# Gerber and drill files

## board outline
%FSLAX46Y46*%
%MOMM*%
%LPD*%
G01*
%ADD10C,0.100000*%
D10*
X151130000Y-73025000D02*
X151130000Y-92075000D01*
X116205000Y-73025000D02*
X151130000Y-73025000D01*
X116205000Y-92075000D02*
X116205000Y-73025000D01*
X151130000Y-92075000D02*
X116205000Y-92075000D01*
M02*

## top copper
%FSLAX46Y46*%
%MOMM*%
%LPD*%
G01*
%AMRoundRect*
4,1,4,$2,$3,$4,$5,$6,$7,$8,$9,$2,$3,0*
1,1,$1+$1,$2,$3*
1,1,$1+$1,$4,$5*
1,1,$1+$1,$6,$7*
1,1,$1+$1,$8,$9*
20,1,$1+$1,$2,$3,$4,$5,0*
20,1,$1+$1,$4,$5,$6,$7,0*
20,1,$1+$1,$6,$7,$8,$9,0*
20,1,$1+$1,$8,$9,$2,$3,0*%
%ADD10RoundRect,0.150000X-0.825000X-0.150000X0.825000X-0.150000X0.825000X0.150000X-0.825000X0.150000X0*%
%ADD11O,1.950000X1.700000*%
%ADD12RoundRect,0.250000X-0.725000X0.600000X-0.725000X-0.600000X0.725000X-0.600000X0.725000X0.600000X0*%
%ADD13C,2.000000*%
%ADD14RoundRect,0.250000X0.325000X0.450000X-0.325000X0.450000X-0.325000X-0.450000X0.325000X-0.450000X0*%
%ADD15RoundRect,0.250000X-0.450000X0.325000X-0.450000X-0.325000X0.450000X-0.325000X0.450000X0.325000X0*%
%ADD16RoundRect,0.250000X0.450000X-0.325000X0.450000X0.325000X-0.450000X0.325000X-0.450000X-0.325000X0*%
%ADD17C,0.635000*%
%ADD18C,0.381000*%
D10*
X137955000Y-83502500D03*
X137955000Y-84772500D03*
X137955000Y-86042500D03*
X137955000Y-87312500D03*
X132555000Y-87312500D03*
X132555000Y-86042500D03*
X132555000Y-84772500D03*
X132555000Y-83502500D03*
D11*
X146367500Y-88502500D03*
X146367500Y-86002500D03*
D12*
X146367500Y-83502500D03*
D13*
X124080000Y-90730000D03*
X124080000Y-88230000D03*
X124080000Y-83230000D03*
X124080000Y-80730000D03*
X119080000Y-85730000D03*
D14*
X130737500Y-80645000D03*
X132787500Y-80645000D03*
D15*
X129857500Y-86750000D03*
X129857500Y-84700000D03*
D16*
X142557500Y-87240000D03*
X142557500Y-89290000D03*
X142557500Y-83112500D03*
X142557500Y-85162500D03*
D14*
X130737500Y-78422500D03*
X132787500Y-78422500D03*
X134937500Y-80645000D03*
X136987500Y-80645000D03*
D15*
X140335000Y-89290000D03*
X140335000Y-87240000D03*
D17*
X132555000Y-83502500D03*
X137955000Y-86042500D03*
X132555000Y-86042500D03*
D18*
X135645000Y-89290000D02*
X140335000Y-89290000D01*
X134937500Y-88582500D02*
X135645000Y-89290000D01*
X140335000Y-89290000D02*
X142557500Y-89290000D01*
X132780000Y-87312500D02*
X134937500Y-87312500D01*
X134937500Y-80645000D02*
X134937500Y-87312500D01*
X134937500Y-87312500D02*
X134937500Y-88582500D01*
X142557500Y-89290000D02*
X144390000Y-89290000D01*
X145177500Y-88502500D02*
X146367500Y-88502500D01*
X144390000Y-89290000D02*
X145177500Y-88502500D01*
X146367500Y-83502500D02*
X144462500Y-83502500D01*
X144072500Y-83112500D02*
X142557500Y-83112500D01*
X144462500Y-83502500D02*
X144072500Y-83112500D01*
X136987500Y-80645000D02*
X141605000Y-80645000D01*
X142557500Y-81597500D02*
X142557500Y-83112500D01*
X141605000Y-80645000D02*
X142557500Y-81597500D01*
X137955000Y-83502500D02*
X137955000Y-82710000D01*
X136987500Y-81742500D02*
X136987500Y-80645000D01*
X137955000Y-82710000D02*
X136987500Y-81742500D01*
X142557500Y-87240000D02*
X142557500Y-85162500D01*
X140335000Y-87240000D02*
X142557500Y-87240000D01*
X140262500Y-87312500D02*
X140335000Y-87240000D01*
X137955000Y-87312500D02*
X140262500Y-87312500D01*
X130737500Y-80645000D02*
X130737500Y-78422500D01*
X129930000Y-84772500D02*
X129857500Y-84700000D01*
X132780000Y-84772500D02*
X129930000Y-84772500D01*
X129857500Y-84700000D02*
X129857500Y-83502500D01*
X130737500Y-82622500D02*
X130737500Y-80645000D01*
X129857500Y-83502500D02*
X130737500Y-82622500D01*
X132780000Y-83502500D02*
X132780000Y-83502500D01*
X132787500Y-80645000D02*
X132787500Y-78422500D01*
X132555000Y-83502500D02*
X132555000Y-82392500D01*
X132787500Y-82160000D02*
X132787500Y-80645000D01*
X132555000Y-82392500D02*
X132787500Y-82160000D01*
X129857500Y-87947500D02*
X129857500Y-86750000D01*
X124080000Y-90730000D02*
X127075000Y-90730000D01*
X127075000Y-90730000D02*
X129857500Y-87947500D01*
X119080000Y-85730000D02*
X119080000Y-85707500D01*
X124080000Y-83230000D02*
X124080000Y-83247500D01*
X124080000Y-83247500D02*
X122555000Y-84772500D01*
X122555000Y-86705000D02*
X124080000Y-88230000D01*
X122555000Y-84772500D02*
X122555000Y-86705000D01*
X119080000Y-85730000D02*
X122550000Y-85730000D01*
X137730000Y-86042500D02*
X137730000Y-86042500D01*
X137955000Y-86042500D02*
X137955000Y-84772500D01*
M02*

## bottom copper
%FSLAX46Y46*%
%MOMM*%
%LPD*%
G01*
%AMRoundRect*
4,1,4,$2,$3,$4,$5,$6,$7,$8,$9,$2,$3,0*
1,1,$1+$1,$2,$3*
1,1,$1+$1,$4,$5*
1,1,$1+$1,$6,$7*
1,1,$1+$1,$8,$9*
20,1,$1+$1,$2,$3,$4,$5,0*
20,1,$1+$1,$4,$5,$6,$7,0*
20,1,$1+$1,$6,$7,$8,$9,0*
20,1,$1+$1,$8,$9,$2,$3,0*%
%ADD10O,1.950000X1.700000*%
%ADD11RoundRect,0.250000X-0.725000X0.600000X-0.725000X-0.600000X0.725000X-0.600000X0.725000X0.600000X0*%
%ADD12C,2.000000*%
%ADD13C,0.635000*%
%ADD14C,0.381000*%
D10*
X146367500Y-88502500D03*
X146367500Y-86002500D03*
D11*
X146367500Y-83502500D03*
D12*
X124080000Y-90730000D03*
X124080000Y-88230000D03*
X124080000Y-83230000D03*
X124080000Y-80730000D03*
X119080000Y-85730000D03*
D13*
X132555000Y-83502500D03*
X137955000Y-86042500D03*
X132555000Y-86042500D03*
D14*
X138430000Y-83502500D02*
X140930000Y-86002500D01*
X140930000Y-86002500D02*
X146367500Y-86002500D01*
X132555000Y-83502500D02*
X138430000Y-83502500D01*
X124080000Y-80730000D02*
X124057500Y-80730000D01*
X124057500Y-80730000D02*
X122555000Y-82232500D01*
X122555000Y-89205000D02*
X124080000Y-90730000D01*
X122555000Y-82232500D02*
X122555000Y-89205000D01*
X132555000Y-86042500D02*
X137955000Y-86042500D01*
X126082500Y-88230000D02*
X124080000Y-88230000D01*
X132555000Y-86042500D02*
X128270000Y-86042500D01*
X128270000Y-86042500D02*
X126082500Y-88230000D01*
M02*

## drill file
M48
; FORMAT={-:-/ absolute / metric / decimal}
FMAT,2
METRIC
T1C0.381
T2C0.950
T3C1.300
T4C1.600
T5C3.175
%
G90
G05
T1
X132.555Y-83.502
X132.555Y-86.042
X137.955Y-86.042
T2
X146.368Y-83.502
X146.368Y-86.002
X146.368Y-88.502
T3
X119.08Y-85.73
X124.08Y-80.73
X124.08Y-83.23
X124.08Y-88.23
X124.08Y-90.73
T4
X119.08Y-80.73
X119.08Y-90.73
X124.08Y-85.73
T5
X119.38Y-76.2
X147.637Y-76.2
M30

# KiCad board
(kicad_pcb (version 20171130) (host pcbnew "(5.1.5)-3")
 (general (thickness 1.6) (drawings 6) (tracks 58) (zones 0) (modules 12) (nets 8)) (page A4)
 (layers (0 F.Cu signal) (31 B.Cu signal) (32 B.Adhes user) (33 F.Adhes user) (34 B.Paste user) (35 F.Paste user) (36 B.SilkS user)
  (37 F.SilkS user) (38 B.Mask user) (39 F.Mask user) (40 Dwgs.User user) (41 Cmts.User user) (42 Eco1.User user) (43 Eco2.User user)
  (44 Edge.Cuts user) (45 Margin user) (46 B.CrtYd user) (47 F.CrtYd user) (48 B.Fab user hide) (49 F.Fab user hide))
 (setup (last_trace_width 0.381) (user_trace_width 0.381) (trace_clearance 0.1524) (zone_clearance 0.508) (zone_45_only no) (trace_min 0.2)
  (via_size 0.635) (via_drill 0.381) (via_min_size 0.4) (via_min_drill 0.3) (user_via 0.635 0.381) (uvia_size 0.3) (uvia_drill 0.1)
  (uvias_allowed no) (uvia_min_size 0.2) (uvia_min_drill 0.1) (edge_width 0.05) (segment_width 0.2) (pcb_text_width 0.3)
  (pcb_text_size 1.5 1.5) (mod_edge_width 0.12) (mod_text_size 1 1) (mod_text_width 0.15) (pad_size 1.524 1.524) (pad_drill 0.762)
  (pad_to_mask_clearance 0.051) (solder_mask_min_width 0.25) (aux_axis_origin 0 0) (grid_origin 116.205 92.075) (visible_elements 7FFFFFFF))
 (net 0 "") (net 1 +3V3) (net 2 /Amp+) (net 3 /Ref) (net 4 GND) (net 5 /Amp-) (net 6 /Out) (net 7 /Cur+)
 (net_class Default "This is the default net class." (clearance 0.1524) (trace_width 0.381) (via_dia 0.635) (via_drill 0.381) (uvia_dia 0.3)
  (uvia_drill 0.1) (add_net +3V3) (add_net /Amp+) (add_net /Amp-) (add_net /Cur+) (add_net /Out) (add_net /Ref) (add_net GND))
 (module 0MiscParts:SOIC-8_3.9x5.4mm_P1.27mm (layer F.Cu) (at 135.255 85.4075)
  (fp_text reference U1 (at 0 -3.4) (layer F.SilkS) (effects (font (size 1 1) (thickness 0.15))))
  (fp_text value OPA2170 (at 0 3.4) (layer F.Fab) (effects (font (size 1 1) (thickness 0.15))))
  (pad 8 smd roundrect (at 2.7 -1.905) (size 1.95 0.6) (layers F.Cu F.Paste F.Mask) (roundrect_rratio 0.25) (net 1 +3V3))
  (pad 7 smd roundrect (at 2.7 -0.635) (size 1.95 0.6) (layers F.Cu F.Paste F.Mask) (roundrect_rratio 0.25) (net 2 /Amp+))
  (pad 6 smd roundrect (at 2.7 0.635) (size 1.95 0.6) (layers F.Cu F.Paste F.Mask) (roundrect_rratio 0.25) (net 2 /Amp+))
  (pad 5 smd roundrect (at 2.7 1.905) (size 1.95 0.6) (layers F.Cu F.Paste F.Mask) (roundrect_rratio 0.25) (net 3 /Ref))
  (pad 4 smd roundrect (at -2.7 1.905) (size 1.95 0.6) (layers F.Cu F.Paste F.Mask) (roundrect_rratio 0.25) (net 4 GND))
  (pad 3 smd roundrect (at -2.7 0.635) (size 1.95 0.6) (layers F.Cu F.Paste F.Mask) (roundrect_rratio 0.25) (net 2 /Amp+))
  (pad 2 smd roundrect (at -2.7 -0.635) (size 1.95 0.6) (layers F.Cu F.Paste F.Mask) (roundrect_rratio 0.25) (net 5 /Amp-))
  (pad 1 smd roundrect (at -2.7 -1.905) (size 1.95 0.6) (layers F.Cu F.Paste F.Mask) (roundrect_rratio 0.25) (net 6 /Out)))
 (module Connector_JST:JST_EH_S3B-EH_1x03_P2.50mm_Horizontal (layer F.Cu) (at 146.3675 83.5025 270)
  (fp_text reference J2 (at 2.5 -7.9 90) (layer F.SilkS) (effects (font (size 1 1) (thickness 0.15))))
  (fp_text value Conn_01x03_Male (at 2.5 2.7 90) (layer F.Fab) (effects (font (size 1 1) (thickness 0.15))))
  (pad 3 thru_hole oval (at 5 0 270) (size 1.7 1.95) (drill 0.95) (layers *.Cu *.Mask) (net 4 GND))
  (pad 2 thru_hole oval (at 2.5 0 270) (size 1.7 1.95) (drill 0.95) (layers *.Cu *.Mask) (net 6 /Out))
  (pad 1 thru_hole roundrect (at 0 0 270) (size 1.7 1.95) (drill 0.95) (layers *.Cu *.Mask) (roundrect_rratio 0.147059) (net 1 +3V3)))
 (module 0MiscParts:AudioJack (layer F.Cu) (at 119.08 85.73)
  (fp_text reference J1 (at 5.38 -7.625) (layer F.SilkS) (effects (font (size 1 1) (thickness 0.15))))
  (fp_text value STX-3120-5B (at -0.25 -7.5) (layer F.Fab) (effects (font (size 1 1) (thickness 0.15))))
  (pad "" np_thru_hole circle (at 5 0) (size 1.6 1.6) (drill 1.6) (layers *.Cu *.Mask))
  (pad "" np_thru_hole circle (at 0 5) (size 1.6 1.6) (drill 1.6) (layers *.Cu *.Mask))
  (pad "" np_thru_hole circle (at 0 -5) (size 1.6 1.6) (drill 1.6) (layers *.Cu *.Mask))
  (pad 5 thru_hole circle (at 5 5) (size 2 2) (drill 1.3) (layers *.Cu *.Mask) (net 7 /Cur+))
  (pad 4 thru_hole circle (at 5 2.5) (size 2 2) (drill 1.3) (layers *.Cu *.Mask) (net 2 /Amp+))
  (pad 3 thru_hole circle (at 5 -2.5) (size 2 2) (drill 1.3) (layers *.Cu *.Mask) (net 2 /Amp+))
  (pad 2 thru_hole circle (at 5 -5) (size 2 2) (drill 1.3) (layers *.Cu *.Mask) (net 7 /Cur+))
  (pad 1 thru_hole circle (at 0 0) (size 2 2) (drill 1.3) (layers *.Cu *.Mask) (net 2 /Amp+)))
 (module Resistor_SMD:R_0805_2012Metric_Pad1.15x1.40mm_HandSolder (layer F.Cu) (at 131.7625 80.645 180)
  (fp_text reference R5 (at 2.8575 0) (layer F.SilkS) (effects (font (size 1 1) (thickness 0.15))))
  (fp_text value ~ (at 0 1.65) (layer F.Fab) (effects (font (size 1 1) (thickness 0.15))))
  (pad 2 smd roundrect (at 1.025 0 180) (size 1.15 1.4) (layers F.Cu F.Paste F.Mask) (roundrect_rratio 0.217391) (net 5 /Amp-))
  (pad 1 smd roundrect (at -1.025 0 180) (size 1.15 1.4) (layers F.Cu F.Paste F.Mask) (roundrect_rratio 0.217391) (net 6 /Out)))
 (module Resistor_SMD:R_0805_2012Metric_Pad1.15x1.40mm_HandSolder (layer F.Cu) (at 129.8575 85.725 270)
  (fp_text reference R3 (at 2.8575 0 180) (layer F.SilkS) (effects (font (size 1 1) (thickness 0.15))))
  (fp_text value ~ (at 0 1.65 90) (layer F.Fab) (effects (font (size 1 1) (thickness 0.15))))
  (pad 2 smd roundrect (at 1.025 0 270) (size 1.15 1.4) (layers F.Cu F.Paste F.Mask) (roundrect_rratio 0.217391) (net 7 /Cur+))
  (pad 1 smd roundrect (at -1.025 0 270) (size 1.15 1.4) (layers F.Cu F.Paste F.Mask) (roundrect_rratio 0.217391) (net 5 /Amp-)))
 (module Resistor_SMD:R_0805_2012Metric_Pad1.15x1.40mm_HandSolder (layer F.Cu) (at 142.5575 88.265 90)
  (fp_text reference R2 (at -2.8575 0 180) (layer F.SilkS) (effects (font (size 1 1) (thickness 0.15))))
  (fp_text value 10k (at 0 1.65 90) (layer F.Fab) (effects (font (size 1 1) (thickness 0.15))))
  (pad 2 smd roundrect (at 1.025 0 90) (size 1.15 1.4) (layers F.Cu F.Paste F.Mask) (roundrect_rratio 0.217391) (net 3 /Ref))
  (pad 1 smd roundrect (at -1.025 0 90) (size 1.15 1.4) (layers F.Cu F.Paste F.Mask) (roundrect_rratio 0.217391) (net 4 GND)))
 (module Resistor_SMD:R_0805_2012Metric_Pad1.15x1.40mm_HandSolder (layer F.Cu) (at 142.5575 84.1375 90)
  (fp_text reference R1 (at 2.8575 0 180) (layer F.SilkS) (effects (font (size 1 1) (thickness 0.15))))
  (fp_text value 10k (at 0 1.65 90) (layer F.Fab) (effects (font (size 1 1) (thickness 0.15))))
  (pad 2 smd roundrect (at 1.025 0 90) (size 1.15 1.4) (layers F.Cu F.Paste F.Mask) (roundrect_rratio 0.217391) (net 1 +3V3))
  (pad 1 smd roundrect (at -1.025 0 90) (size 1.15 1.4) (layers F.Cu F.Paste F.Mask) (roundrect_rratio 0.217391) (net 3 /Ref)))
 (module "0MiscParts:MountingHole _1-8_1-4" (layer F.Cu) (at 147.6375 76.2)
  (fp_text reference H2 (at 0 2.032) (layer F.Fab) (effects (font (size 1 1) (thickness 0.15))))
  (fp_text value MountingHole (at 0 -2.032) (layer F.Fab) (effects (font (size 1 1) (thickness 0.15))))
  (pad "" np_thru_hole circle (at 0 0) (size 3.175 3.175) (drill 3.175) (layers *.Cu *.Mask)))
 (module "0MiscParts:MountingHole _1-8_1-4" (layer F.Cu) (at 119.38 76.2)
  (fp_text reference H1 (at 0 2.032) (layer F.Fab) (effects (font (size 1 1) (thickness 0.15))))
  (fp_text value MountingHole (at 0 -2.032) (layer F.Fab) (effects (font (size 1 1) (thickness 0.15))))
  (pad "" np_thru_hole circle (at 0 0) (size 3.175 3.175) (drill 3.175) (layers *.Cu *.Mask)))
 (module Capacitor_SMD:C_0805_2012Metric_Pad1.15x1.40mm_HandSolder (layer F.Cu) (at 131.7625 78.4225 180)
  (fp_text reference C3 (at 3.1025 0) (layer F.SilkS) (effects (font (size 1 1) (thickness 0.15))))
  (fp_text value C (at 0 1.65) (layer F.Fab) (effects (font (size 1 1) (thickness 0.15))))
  (pad 2 smd roundrect (at 1.025 0 180) (size 1.15 1.4) (layers F.Cu F.Paste F.Mask) (roundrect_rratio 0.217391) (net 5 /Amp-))
  (pad 1 smd roundrect (at -1.025 0 180) (size 1.15 1.4) (layers F.Cu F.Paste F.Mask) (roundrect_rratio 0.217391) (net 6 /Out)))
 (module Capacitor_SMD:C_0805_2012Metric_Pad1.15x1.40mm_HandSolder (layer F.Cu) (at 135.9625 80.645 180)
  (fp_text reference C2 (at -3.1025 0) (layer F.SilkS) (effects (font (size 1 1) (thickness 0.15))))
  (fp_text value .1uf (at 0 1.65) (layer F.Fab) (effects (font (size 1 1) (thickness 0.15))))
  (pad 2 smd roundrect (at 1.025 0 180) (size 1.15 1.4) (layers F.Cu F.Paste F.Mask) (roundrect_rratio 0.217391) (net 4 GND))
  (pad 1 smd roundrect (at -1.025 0 180) (size 1.15 1.4) (layers F.Cu F.Paste F.Mask) (roundrect_rratio 0.217391) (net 1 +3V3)))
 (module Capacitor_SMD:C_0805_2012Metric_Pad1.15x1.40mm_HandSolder (layer F.Cu) (at 140.335 88.265 270)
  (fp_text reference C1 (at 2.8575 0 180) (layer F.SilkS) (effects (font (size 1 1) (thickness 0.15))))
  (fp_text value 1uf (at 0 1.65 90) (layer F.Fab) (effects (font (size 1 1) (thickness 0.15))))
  (pad 2 smd roundrect (at 1.025 0 270) (size 1.15 1.4) (layers F.Cu F.Paste F.Mask) (roundrect_rratio 0.217391) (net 4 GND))
  (pad 1 smd roundrect (at -1.025 0 270) (size 1.15 1.4) (layers F.Cu F.Paste F.Mask) (roundrect_rratio 0.217391) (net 3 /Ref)))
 (gr_line (start 151.13 73.025) (end 151.13 92.075) (layer Edge.Cuts) (width 0.1))
 (gr_line (start 116.205 73.025) (end 151.13 73.025) (layer Edge.Cuts) (width 0.1))
 (gr_line (start 116.205 92.075) (end 116.205 73.025) (layer Edge.Cuts) (width 0.1))
 (gr_line (start 151.13 92.075) (end 116.205 92.075) (layer Edge.Cuts) (width 0.1))
 (segment (start 135.645 89.29) (end 140.335 89.29) (width 0.381) (layer F.Cu) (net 4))
 (segment (start 134.9375 88.5825) (end 135.645 89.29) (width 0.381) (layer F.Cu) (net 4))
 (segment (start 140.335 89.29) (end 142.5575 89.29) (width 0.381) (layer F.Cu) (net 4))
 (segment (start 132.78 87.3125) (end 134.9375 87.3125) (width 0.381) (layer F.Cu) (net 4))
 (segment (start 134.9375 80.645) (end 134.9375 87.3125) (width 0.381) (layer F.Cu) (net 4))
 (segment (start 134.9375 87.3125) (end 134.9375 88.5825) (width 0.381) (layer F.Cu) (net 4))
 (segment (start 142.5575 89.29) (end 144.39 89.29) (width 0.381) (layer F.Cu) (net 4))
 (segment (start 145.1775 88.5025) (end 146.3675 88.5025) (width 0.381) (layer F.Cu) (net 4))
 (segment (start 144.39 89.29) (end 145.1775 88.5025) (width 0.381) (layer F.Cu) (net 4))
 (segment (start 146.3675 83.5025) (end 144.4625 83.5025) (width 0.381) (layer F.Cu) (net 1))
 (segment (start 144.0725 83.1125) (end 142.5575 83.1125) (width 0.381) (layer F.Cu) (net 1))
 (segment (start 144.4625 83.5025) (end 144.0725 83.1125) (width 0.381) (layer F.Cu) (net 1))
 (segment (start 136.9875 80.645) (end 141.605 80.645) (width 0.381) (layer F.Cu) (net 1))
 (segment (start 142.5575 81.5975) (end 142.5575 83.1125) (width 0.381) (layer F.Cu) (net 1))
 (segment (start 141.605 80.645) (end 142.5575 81.5975) (width 0.381) (layer F.Cu) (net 1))
 (segment (start 137.955 83.5025) (end 137.955 82.71) (width 0.381) (layer F.Cu) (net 1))
 (segment (start 136.9875 81.7425) (end 136.9875 80.645) (width 0.381) (layer F.Cu) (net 1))
 (segment (start 137.955 82.71) (end 136.9875 81.7425) (width 0.381) (layer F.Cu) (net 1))
 (segment (start 142.5575 87.24) (end 142.5575 85.1625) (width 0.381) (layer F.Cu) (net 3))
 (segment (start 140.335 87.24) (end 142.5575 87.24) (width 0.381) (layer F.Cu) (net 3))
 (segment (start 140.2625 87.3125) (end 140.335 87.24) (width 0.381) (layer F.Cu) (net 3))
 (segment (start 137.955 87.3125) (end 140.2625 87.3125) (width 0.381) (layer F.Cu) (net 3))
 (segment (start 130.7375 80.645) (end 130.7375 78.4225) (width 0.381) (layer F.Cu) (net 5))
 (segment (start 129.93 84.7725) (end 129.8575 84.7) (width 0.381) (layer F.Cu) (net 5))
 (segment (start 132.78 84.7725) (end 129.93 84.7725) (width 0.381) (layer F.Cu) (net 5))
 (segment (start 129.8575 84.7) (end 129.8575 83.5025) (width 0.381) (layer F.Cu) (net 5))
 (segment (start 130.7375 82.6225) (end 130.7375 80.645) (width 0.381) (layer F.Cu) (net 5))
 (segment (start 129.8575 83.5025) (end 130.7375 82.6225) (width 0.381) (layer F.Cu) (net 5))
 (segment (start 132.78 83.5025) (end 132.78 83.5025) (width 0.381) (layer F.Cu) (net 6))
 (segment (start 132.7875 80.645) (end 132.7875 78.4225) (width 0.381) (layer F.Cu) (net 6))
 (segment (start 138.43 83.5025) (end 140.93 86.0025) (width 0.381) (layer B.Cu) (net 6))
 (via (at 132.555 83.5025) (size 0.635) (drill 0.381) (layers F.Cu B.Cu) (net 6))
 (segment (start 140.93 86.0025) (end 146.3675 86.0025) (width 0.381) (layer B.Cu) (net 6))
 (segment (start 132.555 83.5025) (end 138.43 83.5025) (width 0.381) (layer B.Cu) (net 6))
 (segment (start 132.555 83.5025) (end 132.555 82.3925) (width 0.381) (layer F.Cu) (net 6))
 (segment (start 132.7875 82.16) (end 132.7875 80.645) (width 0.381) (layer F.Cu) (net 6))
 (segment (start 132.555 82.3925) (end 132.7875 82.16) (width 0.381) (layer F.Cu) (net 6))
 (segment (start 124.08 80.73) (end 124.0575 80.73) (width 0.381) (layer B.Cu) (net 7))
 (segment (start 124.0575 80.73) (end 122.555 82.2325) (width 0.381) (layer B.Cu) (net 7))
 (segment (start 122.555 89.205) (end 124.08 90.73) (width 0.381) (layer B.Cu) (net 7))
 (segment (start 122.555 82.2325) (end 122.555 89.205) (width 0.381) (layer B.Cu) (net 7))
 (segment (start 129.8575 87.9475) (end 129.8575 86.75) (width 0.381) (layer F.Cu) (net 7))
 (segment (start 124.08 90.73) (end 127.075 90.73) (width 0.381) (layer F.Cu) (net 7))
 (segment (start 127.075 90.73) (end 129.8575 87.9475) (width 0.381) (layer F.Cu) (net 7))
 (segment (start 119.08 85.73) (end 119.08 85.7075) (width 0.381) (layer F.Cu) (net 2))
 (segment (start 124.08 83.23) (end 124.08 83.2475) (width 0.381) (layer F.Cu) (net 2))
 (segment (start 124.08 83.2475) (end 122.555 84.7725) (width 0.381) (layer F.Cu) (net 2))
 (segment (start 122.555 86.705) (end 124.08 88.23) (width 0.381) (layer F.Cu) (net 2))
 (segment (start 122.555 84.7725) (end 122.555 86.705) (width 0.381) (layer F.Cu) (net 2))
 (segment (start 119.08 85.73) (end 122.55 85.73) (width 0.381) (layer F.Cu) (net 2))
 (segment (start 137.73 86.0425) (end 137.73 86.0425) (width 0.381) (layer F.Cu) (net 2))
 (via (at 137.955 86.0425) (size 0.635) (drill 0.381) (layers F.Cu B.Cu) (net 2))
 (via (at 132.555 86.0425) (size 0.635) (drill 0.381) (layers F.Cu B.Cu) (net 2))
 (segment (start 132.555 86.0425) (end 137.955 86.0425) (width 0.381) (layer B.Cu) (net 2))
 (segment (start 137.955 86.0425) (end 137.955 84.7725) (width 0.381) (layer F.Cu) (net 2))
 (segment (start 126.0825 88.23) (end 124.08 88.23) (width 0.381) (layer B.Cu) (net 2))
 (segment (start 132.555 86.0425) (end 128.27 86.0425) (width 0.381) (layer B.Cu) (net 2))
 (segment (start 128.27 86.0425) (end 126.0825 88.23) (width 0.381) (layer B.Cu) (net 2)))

